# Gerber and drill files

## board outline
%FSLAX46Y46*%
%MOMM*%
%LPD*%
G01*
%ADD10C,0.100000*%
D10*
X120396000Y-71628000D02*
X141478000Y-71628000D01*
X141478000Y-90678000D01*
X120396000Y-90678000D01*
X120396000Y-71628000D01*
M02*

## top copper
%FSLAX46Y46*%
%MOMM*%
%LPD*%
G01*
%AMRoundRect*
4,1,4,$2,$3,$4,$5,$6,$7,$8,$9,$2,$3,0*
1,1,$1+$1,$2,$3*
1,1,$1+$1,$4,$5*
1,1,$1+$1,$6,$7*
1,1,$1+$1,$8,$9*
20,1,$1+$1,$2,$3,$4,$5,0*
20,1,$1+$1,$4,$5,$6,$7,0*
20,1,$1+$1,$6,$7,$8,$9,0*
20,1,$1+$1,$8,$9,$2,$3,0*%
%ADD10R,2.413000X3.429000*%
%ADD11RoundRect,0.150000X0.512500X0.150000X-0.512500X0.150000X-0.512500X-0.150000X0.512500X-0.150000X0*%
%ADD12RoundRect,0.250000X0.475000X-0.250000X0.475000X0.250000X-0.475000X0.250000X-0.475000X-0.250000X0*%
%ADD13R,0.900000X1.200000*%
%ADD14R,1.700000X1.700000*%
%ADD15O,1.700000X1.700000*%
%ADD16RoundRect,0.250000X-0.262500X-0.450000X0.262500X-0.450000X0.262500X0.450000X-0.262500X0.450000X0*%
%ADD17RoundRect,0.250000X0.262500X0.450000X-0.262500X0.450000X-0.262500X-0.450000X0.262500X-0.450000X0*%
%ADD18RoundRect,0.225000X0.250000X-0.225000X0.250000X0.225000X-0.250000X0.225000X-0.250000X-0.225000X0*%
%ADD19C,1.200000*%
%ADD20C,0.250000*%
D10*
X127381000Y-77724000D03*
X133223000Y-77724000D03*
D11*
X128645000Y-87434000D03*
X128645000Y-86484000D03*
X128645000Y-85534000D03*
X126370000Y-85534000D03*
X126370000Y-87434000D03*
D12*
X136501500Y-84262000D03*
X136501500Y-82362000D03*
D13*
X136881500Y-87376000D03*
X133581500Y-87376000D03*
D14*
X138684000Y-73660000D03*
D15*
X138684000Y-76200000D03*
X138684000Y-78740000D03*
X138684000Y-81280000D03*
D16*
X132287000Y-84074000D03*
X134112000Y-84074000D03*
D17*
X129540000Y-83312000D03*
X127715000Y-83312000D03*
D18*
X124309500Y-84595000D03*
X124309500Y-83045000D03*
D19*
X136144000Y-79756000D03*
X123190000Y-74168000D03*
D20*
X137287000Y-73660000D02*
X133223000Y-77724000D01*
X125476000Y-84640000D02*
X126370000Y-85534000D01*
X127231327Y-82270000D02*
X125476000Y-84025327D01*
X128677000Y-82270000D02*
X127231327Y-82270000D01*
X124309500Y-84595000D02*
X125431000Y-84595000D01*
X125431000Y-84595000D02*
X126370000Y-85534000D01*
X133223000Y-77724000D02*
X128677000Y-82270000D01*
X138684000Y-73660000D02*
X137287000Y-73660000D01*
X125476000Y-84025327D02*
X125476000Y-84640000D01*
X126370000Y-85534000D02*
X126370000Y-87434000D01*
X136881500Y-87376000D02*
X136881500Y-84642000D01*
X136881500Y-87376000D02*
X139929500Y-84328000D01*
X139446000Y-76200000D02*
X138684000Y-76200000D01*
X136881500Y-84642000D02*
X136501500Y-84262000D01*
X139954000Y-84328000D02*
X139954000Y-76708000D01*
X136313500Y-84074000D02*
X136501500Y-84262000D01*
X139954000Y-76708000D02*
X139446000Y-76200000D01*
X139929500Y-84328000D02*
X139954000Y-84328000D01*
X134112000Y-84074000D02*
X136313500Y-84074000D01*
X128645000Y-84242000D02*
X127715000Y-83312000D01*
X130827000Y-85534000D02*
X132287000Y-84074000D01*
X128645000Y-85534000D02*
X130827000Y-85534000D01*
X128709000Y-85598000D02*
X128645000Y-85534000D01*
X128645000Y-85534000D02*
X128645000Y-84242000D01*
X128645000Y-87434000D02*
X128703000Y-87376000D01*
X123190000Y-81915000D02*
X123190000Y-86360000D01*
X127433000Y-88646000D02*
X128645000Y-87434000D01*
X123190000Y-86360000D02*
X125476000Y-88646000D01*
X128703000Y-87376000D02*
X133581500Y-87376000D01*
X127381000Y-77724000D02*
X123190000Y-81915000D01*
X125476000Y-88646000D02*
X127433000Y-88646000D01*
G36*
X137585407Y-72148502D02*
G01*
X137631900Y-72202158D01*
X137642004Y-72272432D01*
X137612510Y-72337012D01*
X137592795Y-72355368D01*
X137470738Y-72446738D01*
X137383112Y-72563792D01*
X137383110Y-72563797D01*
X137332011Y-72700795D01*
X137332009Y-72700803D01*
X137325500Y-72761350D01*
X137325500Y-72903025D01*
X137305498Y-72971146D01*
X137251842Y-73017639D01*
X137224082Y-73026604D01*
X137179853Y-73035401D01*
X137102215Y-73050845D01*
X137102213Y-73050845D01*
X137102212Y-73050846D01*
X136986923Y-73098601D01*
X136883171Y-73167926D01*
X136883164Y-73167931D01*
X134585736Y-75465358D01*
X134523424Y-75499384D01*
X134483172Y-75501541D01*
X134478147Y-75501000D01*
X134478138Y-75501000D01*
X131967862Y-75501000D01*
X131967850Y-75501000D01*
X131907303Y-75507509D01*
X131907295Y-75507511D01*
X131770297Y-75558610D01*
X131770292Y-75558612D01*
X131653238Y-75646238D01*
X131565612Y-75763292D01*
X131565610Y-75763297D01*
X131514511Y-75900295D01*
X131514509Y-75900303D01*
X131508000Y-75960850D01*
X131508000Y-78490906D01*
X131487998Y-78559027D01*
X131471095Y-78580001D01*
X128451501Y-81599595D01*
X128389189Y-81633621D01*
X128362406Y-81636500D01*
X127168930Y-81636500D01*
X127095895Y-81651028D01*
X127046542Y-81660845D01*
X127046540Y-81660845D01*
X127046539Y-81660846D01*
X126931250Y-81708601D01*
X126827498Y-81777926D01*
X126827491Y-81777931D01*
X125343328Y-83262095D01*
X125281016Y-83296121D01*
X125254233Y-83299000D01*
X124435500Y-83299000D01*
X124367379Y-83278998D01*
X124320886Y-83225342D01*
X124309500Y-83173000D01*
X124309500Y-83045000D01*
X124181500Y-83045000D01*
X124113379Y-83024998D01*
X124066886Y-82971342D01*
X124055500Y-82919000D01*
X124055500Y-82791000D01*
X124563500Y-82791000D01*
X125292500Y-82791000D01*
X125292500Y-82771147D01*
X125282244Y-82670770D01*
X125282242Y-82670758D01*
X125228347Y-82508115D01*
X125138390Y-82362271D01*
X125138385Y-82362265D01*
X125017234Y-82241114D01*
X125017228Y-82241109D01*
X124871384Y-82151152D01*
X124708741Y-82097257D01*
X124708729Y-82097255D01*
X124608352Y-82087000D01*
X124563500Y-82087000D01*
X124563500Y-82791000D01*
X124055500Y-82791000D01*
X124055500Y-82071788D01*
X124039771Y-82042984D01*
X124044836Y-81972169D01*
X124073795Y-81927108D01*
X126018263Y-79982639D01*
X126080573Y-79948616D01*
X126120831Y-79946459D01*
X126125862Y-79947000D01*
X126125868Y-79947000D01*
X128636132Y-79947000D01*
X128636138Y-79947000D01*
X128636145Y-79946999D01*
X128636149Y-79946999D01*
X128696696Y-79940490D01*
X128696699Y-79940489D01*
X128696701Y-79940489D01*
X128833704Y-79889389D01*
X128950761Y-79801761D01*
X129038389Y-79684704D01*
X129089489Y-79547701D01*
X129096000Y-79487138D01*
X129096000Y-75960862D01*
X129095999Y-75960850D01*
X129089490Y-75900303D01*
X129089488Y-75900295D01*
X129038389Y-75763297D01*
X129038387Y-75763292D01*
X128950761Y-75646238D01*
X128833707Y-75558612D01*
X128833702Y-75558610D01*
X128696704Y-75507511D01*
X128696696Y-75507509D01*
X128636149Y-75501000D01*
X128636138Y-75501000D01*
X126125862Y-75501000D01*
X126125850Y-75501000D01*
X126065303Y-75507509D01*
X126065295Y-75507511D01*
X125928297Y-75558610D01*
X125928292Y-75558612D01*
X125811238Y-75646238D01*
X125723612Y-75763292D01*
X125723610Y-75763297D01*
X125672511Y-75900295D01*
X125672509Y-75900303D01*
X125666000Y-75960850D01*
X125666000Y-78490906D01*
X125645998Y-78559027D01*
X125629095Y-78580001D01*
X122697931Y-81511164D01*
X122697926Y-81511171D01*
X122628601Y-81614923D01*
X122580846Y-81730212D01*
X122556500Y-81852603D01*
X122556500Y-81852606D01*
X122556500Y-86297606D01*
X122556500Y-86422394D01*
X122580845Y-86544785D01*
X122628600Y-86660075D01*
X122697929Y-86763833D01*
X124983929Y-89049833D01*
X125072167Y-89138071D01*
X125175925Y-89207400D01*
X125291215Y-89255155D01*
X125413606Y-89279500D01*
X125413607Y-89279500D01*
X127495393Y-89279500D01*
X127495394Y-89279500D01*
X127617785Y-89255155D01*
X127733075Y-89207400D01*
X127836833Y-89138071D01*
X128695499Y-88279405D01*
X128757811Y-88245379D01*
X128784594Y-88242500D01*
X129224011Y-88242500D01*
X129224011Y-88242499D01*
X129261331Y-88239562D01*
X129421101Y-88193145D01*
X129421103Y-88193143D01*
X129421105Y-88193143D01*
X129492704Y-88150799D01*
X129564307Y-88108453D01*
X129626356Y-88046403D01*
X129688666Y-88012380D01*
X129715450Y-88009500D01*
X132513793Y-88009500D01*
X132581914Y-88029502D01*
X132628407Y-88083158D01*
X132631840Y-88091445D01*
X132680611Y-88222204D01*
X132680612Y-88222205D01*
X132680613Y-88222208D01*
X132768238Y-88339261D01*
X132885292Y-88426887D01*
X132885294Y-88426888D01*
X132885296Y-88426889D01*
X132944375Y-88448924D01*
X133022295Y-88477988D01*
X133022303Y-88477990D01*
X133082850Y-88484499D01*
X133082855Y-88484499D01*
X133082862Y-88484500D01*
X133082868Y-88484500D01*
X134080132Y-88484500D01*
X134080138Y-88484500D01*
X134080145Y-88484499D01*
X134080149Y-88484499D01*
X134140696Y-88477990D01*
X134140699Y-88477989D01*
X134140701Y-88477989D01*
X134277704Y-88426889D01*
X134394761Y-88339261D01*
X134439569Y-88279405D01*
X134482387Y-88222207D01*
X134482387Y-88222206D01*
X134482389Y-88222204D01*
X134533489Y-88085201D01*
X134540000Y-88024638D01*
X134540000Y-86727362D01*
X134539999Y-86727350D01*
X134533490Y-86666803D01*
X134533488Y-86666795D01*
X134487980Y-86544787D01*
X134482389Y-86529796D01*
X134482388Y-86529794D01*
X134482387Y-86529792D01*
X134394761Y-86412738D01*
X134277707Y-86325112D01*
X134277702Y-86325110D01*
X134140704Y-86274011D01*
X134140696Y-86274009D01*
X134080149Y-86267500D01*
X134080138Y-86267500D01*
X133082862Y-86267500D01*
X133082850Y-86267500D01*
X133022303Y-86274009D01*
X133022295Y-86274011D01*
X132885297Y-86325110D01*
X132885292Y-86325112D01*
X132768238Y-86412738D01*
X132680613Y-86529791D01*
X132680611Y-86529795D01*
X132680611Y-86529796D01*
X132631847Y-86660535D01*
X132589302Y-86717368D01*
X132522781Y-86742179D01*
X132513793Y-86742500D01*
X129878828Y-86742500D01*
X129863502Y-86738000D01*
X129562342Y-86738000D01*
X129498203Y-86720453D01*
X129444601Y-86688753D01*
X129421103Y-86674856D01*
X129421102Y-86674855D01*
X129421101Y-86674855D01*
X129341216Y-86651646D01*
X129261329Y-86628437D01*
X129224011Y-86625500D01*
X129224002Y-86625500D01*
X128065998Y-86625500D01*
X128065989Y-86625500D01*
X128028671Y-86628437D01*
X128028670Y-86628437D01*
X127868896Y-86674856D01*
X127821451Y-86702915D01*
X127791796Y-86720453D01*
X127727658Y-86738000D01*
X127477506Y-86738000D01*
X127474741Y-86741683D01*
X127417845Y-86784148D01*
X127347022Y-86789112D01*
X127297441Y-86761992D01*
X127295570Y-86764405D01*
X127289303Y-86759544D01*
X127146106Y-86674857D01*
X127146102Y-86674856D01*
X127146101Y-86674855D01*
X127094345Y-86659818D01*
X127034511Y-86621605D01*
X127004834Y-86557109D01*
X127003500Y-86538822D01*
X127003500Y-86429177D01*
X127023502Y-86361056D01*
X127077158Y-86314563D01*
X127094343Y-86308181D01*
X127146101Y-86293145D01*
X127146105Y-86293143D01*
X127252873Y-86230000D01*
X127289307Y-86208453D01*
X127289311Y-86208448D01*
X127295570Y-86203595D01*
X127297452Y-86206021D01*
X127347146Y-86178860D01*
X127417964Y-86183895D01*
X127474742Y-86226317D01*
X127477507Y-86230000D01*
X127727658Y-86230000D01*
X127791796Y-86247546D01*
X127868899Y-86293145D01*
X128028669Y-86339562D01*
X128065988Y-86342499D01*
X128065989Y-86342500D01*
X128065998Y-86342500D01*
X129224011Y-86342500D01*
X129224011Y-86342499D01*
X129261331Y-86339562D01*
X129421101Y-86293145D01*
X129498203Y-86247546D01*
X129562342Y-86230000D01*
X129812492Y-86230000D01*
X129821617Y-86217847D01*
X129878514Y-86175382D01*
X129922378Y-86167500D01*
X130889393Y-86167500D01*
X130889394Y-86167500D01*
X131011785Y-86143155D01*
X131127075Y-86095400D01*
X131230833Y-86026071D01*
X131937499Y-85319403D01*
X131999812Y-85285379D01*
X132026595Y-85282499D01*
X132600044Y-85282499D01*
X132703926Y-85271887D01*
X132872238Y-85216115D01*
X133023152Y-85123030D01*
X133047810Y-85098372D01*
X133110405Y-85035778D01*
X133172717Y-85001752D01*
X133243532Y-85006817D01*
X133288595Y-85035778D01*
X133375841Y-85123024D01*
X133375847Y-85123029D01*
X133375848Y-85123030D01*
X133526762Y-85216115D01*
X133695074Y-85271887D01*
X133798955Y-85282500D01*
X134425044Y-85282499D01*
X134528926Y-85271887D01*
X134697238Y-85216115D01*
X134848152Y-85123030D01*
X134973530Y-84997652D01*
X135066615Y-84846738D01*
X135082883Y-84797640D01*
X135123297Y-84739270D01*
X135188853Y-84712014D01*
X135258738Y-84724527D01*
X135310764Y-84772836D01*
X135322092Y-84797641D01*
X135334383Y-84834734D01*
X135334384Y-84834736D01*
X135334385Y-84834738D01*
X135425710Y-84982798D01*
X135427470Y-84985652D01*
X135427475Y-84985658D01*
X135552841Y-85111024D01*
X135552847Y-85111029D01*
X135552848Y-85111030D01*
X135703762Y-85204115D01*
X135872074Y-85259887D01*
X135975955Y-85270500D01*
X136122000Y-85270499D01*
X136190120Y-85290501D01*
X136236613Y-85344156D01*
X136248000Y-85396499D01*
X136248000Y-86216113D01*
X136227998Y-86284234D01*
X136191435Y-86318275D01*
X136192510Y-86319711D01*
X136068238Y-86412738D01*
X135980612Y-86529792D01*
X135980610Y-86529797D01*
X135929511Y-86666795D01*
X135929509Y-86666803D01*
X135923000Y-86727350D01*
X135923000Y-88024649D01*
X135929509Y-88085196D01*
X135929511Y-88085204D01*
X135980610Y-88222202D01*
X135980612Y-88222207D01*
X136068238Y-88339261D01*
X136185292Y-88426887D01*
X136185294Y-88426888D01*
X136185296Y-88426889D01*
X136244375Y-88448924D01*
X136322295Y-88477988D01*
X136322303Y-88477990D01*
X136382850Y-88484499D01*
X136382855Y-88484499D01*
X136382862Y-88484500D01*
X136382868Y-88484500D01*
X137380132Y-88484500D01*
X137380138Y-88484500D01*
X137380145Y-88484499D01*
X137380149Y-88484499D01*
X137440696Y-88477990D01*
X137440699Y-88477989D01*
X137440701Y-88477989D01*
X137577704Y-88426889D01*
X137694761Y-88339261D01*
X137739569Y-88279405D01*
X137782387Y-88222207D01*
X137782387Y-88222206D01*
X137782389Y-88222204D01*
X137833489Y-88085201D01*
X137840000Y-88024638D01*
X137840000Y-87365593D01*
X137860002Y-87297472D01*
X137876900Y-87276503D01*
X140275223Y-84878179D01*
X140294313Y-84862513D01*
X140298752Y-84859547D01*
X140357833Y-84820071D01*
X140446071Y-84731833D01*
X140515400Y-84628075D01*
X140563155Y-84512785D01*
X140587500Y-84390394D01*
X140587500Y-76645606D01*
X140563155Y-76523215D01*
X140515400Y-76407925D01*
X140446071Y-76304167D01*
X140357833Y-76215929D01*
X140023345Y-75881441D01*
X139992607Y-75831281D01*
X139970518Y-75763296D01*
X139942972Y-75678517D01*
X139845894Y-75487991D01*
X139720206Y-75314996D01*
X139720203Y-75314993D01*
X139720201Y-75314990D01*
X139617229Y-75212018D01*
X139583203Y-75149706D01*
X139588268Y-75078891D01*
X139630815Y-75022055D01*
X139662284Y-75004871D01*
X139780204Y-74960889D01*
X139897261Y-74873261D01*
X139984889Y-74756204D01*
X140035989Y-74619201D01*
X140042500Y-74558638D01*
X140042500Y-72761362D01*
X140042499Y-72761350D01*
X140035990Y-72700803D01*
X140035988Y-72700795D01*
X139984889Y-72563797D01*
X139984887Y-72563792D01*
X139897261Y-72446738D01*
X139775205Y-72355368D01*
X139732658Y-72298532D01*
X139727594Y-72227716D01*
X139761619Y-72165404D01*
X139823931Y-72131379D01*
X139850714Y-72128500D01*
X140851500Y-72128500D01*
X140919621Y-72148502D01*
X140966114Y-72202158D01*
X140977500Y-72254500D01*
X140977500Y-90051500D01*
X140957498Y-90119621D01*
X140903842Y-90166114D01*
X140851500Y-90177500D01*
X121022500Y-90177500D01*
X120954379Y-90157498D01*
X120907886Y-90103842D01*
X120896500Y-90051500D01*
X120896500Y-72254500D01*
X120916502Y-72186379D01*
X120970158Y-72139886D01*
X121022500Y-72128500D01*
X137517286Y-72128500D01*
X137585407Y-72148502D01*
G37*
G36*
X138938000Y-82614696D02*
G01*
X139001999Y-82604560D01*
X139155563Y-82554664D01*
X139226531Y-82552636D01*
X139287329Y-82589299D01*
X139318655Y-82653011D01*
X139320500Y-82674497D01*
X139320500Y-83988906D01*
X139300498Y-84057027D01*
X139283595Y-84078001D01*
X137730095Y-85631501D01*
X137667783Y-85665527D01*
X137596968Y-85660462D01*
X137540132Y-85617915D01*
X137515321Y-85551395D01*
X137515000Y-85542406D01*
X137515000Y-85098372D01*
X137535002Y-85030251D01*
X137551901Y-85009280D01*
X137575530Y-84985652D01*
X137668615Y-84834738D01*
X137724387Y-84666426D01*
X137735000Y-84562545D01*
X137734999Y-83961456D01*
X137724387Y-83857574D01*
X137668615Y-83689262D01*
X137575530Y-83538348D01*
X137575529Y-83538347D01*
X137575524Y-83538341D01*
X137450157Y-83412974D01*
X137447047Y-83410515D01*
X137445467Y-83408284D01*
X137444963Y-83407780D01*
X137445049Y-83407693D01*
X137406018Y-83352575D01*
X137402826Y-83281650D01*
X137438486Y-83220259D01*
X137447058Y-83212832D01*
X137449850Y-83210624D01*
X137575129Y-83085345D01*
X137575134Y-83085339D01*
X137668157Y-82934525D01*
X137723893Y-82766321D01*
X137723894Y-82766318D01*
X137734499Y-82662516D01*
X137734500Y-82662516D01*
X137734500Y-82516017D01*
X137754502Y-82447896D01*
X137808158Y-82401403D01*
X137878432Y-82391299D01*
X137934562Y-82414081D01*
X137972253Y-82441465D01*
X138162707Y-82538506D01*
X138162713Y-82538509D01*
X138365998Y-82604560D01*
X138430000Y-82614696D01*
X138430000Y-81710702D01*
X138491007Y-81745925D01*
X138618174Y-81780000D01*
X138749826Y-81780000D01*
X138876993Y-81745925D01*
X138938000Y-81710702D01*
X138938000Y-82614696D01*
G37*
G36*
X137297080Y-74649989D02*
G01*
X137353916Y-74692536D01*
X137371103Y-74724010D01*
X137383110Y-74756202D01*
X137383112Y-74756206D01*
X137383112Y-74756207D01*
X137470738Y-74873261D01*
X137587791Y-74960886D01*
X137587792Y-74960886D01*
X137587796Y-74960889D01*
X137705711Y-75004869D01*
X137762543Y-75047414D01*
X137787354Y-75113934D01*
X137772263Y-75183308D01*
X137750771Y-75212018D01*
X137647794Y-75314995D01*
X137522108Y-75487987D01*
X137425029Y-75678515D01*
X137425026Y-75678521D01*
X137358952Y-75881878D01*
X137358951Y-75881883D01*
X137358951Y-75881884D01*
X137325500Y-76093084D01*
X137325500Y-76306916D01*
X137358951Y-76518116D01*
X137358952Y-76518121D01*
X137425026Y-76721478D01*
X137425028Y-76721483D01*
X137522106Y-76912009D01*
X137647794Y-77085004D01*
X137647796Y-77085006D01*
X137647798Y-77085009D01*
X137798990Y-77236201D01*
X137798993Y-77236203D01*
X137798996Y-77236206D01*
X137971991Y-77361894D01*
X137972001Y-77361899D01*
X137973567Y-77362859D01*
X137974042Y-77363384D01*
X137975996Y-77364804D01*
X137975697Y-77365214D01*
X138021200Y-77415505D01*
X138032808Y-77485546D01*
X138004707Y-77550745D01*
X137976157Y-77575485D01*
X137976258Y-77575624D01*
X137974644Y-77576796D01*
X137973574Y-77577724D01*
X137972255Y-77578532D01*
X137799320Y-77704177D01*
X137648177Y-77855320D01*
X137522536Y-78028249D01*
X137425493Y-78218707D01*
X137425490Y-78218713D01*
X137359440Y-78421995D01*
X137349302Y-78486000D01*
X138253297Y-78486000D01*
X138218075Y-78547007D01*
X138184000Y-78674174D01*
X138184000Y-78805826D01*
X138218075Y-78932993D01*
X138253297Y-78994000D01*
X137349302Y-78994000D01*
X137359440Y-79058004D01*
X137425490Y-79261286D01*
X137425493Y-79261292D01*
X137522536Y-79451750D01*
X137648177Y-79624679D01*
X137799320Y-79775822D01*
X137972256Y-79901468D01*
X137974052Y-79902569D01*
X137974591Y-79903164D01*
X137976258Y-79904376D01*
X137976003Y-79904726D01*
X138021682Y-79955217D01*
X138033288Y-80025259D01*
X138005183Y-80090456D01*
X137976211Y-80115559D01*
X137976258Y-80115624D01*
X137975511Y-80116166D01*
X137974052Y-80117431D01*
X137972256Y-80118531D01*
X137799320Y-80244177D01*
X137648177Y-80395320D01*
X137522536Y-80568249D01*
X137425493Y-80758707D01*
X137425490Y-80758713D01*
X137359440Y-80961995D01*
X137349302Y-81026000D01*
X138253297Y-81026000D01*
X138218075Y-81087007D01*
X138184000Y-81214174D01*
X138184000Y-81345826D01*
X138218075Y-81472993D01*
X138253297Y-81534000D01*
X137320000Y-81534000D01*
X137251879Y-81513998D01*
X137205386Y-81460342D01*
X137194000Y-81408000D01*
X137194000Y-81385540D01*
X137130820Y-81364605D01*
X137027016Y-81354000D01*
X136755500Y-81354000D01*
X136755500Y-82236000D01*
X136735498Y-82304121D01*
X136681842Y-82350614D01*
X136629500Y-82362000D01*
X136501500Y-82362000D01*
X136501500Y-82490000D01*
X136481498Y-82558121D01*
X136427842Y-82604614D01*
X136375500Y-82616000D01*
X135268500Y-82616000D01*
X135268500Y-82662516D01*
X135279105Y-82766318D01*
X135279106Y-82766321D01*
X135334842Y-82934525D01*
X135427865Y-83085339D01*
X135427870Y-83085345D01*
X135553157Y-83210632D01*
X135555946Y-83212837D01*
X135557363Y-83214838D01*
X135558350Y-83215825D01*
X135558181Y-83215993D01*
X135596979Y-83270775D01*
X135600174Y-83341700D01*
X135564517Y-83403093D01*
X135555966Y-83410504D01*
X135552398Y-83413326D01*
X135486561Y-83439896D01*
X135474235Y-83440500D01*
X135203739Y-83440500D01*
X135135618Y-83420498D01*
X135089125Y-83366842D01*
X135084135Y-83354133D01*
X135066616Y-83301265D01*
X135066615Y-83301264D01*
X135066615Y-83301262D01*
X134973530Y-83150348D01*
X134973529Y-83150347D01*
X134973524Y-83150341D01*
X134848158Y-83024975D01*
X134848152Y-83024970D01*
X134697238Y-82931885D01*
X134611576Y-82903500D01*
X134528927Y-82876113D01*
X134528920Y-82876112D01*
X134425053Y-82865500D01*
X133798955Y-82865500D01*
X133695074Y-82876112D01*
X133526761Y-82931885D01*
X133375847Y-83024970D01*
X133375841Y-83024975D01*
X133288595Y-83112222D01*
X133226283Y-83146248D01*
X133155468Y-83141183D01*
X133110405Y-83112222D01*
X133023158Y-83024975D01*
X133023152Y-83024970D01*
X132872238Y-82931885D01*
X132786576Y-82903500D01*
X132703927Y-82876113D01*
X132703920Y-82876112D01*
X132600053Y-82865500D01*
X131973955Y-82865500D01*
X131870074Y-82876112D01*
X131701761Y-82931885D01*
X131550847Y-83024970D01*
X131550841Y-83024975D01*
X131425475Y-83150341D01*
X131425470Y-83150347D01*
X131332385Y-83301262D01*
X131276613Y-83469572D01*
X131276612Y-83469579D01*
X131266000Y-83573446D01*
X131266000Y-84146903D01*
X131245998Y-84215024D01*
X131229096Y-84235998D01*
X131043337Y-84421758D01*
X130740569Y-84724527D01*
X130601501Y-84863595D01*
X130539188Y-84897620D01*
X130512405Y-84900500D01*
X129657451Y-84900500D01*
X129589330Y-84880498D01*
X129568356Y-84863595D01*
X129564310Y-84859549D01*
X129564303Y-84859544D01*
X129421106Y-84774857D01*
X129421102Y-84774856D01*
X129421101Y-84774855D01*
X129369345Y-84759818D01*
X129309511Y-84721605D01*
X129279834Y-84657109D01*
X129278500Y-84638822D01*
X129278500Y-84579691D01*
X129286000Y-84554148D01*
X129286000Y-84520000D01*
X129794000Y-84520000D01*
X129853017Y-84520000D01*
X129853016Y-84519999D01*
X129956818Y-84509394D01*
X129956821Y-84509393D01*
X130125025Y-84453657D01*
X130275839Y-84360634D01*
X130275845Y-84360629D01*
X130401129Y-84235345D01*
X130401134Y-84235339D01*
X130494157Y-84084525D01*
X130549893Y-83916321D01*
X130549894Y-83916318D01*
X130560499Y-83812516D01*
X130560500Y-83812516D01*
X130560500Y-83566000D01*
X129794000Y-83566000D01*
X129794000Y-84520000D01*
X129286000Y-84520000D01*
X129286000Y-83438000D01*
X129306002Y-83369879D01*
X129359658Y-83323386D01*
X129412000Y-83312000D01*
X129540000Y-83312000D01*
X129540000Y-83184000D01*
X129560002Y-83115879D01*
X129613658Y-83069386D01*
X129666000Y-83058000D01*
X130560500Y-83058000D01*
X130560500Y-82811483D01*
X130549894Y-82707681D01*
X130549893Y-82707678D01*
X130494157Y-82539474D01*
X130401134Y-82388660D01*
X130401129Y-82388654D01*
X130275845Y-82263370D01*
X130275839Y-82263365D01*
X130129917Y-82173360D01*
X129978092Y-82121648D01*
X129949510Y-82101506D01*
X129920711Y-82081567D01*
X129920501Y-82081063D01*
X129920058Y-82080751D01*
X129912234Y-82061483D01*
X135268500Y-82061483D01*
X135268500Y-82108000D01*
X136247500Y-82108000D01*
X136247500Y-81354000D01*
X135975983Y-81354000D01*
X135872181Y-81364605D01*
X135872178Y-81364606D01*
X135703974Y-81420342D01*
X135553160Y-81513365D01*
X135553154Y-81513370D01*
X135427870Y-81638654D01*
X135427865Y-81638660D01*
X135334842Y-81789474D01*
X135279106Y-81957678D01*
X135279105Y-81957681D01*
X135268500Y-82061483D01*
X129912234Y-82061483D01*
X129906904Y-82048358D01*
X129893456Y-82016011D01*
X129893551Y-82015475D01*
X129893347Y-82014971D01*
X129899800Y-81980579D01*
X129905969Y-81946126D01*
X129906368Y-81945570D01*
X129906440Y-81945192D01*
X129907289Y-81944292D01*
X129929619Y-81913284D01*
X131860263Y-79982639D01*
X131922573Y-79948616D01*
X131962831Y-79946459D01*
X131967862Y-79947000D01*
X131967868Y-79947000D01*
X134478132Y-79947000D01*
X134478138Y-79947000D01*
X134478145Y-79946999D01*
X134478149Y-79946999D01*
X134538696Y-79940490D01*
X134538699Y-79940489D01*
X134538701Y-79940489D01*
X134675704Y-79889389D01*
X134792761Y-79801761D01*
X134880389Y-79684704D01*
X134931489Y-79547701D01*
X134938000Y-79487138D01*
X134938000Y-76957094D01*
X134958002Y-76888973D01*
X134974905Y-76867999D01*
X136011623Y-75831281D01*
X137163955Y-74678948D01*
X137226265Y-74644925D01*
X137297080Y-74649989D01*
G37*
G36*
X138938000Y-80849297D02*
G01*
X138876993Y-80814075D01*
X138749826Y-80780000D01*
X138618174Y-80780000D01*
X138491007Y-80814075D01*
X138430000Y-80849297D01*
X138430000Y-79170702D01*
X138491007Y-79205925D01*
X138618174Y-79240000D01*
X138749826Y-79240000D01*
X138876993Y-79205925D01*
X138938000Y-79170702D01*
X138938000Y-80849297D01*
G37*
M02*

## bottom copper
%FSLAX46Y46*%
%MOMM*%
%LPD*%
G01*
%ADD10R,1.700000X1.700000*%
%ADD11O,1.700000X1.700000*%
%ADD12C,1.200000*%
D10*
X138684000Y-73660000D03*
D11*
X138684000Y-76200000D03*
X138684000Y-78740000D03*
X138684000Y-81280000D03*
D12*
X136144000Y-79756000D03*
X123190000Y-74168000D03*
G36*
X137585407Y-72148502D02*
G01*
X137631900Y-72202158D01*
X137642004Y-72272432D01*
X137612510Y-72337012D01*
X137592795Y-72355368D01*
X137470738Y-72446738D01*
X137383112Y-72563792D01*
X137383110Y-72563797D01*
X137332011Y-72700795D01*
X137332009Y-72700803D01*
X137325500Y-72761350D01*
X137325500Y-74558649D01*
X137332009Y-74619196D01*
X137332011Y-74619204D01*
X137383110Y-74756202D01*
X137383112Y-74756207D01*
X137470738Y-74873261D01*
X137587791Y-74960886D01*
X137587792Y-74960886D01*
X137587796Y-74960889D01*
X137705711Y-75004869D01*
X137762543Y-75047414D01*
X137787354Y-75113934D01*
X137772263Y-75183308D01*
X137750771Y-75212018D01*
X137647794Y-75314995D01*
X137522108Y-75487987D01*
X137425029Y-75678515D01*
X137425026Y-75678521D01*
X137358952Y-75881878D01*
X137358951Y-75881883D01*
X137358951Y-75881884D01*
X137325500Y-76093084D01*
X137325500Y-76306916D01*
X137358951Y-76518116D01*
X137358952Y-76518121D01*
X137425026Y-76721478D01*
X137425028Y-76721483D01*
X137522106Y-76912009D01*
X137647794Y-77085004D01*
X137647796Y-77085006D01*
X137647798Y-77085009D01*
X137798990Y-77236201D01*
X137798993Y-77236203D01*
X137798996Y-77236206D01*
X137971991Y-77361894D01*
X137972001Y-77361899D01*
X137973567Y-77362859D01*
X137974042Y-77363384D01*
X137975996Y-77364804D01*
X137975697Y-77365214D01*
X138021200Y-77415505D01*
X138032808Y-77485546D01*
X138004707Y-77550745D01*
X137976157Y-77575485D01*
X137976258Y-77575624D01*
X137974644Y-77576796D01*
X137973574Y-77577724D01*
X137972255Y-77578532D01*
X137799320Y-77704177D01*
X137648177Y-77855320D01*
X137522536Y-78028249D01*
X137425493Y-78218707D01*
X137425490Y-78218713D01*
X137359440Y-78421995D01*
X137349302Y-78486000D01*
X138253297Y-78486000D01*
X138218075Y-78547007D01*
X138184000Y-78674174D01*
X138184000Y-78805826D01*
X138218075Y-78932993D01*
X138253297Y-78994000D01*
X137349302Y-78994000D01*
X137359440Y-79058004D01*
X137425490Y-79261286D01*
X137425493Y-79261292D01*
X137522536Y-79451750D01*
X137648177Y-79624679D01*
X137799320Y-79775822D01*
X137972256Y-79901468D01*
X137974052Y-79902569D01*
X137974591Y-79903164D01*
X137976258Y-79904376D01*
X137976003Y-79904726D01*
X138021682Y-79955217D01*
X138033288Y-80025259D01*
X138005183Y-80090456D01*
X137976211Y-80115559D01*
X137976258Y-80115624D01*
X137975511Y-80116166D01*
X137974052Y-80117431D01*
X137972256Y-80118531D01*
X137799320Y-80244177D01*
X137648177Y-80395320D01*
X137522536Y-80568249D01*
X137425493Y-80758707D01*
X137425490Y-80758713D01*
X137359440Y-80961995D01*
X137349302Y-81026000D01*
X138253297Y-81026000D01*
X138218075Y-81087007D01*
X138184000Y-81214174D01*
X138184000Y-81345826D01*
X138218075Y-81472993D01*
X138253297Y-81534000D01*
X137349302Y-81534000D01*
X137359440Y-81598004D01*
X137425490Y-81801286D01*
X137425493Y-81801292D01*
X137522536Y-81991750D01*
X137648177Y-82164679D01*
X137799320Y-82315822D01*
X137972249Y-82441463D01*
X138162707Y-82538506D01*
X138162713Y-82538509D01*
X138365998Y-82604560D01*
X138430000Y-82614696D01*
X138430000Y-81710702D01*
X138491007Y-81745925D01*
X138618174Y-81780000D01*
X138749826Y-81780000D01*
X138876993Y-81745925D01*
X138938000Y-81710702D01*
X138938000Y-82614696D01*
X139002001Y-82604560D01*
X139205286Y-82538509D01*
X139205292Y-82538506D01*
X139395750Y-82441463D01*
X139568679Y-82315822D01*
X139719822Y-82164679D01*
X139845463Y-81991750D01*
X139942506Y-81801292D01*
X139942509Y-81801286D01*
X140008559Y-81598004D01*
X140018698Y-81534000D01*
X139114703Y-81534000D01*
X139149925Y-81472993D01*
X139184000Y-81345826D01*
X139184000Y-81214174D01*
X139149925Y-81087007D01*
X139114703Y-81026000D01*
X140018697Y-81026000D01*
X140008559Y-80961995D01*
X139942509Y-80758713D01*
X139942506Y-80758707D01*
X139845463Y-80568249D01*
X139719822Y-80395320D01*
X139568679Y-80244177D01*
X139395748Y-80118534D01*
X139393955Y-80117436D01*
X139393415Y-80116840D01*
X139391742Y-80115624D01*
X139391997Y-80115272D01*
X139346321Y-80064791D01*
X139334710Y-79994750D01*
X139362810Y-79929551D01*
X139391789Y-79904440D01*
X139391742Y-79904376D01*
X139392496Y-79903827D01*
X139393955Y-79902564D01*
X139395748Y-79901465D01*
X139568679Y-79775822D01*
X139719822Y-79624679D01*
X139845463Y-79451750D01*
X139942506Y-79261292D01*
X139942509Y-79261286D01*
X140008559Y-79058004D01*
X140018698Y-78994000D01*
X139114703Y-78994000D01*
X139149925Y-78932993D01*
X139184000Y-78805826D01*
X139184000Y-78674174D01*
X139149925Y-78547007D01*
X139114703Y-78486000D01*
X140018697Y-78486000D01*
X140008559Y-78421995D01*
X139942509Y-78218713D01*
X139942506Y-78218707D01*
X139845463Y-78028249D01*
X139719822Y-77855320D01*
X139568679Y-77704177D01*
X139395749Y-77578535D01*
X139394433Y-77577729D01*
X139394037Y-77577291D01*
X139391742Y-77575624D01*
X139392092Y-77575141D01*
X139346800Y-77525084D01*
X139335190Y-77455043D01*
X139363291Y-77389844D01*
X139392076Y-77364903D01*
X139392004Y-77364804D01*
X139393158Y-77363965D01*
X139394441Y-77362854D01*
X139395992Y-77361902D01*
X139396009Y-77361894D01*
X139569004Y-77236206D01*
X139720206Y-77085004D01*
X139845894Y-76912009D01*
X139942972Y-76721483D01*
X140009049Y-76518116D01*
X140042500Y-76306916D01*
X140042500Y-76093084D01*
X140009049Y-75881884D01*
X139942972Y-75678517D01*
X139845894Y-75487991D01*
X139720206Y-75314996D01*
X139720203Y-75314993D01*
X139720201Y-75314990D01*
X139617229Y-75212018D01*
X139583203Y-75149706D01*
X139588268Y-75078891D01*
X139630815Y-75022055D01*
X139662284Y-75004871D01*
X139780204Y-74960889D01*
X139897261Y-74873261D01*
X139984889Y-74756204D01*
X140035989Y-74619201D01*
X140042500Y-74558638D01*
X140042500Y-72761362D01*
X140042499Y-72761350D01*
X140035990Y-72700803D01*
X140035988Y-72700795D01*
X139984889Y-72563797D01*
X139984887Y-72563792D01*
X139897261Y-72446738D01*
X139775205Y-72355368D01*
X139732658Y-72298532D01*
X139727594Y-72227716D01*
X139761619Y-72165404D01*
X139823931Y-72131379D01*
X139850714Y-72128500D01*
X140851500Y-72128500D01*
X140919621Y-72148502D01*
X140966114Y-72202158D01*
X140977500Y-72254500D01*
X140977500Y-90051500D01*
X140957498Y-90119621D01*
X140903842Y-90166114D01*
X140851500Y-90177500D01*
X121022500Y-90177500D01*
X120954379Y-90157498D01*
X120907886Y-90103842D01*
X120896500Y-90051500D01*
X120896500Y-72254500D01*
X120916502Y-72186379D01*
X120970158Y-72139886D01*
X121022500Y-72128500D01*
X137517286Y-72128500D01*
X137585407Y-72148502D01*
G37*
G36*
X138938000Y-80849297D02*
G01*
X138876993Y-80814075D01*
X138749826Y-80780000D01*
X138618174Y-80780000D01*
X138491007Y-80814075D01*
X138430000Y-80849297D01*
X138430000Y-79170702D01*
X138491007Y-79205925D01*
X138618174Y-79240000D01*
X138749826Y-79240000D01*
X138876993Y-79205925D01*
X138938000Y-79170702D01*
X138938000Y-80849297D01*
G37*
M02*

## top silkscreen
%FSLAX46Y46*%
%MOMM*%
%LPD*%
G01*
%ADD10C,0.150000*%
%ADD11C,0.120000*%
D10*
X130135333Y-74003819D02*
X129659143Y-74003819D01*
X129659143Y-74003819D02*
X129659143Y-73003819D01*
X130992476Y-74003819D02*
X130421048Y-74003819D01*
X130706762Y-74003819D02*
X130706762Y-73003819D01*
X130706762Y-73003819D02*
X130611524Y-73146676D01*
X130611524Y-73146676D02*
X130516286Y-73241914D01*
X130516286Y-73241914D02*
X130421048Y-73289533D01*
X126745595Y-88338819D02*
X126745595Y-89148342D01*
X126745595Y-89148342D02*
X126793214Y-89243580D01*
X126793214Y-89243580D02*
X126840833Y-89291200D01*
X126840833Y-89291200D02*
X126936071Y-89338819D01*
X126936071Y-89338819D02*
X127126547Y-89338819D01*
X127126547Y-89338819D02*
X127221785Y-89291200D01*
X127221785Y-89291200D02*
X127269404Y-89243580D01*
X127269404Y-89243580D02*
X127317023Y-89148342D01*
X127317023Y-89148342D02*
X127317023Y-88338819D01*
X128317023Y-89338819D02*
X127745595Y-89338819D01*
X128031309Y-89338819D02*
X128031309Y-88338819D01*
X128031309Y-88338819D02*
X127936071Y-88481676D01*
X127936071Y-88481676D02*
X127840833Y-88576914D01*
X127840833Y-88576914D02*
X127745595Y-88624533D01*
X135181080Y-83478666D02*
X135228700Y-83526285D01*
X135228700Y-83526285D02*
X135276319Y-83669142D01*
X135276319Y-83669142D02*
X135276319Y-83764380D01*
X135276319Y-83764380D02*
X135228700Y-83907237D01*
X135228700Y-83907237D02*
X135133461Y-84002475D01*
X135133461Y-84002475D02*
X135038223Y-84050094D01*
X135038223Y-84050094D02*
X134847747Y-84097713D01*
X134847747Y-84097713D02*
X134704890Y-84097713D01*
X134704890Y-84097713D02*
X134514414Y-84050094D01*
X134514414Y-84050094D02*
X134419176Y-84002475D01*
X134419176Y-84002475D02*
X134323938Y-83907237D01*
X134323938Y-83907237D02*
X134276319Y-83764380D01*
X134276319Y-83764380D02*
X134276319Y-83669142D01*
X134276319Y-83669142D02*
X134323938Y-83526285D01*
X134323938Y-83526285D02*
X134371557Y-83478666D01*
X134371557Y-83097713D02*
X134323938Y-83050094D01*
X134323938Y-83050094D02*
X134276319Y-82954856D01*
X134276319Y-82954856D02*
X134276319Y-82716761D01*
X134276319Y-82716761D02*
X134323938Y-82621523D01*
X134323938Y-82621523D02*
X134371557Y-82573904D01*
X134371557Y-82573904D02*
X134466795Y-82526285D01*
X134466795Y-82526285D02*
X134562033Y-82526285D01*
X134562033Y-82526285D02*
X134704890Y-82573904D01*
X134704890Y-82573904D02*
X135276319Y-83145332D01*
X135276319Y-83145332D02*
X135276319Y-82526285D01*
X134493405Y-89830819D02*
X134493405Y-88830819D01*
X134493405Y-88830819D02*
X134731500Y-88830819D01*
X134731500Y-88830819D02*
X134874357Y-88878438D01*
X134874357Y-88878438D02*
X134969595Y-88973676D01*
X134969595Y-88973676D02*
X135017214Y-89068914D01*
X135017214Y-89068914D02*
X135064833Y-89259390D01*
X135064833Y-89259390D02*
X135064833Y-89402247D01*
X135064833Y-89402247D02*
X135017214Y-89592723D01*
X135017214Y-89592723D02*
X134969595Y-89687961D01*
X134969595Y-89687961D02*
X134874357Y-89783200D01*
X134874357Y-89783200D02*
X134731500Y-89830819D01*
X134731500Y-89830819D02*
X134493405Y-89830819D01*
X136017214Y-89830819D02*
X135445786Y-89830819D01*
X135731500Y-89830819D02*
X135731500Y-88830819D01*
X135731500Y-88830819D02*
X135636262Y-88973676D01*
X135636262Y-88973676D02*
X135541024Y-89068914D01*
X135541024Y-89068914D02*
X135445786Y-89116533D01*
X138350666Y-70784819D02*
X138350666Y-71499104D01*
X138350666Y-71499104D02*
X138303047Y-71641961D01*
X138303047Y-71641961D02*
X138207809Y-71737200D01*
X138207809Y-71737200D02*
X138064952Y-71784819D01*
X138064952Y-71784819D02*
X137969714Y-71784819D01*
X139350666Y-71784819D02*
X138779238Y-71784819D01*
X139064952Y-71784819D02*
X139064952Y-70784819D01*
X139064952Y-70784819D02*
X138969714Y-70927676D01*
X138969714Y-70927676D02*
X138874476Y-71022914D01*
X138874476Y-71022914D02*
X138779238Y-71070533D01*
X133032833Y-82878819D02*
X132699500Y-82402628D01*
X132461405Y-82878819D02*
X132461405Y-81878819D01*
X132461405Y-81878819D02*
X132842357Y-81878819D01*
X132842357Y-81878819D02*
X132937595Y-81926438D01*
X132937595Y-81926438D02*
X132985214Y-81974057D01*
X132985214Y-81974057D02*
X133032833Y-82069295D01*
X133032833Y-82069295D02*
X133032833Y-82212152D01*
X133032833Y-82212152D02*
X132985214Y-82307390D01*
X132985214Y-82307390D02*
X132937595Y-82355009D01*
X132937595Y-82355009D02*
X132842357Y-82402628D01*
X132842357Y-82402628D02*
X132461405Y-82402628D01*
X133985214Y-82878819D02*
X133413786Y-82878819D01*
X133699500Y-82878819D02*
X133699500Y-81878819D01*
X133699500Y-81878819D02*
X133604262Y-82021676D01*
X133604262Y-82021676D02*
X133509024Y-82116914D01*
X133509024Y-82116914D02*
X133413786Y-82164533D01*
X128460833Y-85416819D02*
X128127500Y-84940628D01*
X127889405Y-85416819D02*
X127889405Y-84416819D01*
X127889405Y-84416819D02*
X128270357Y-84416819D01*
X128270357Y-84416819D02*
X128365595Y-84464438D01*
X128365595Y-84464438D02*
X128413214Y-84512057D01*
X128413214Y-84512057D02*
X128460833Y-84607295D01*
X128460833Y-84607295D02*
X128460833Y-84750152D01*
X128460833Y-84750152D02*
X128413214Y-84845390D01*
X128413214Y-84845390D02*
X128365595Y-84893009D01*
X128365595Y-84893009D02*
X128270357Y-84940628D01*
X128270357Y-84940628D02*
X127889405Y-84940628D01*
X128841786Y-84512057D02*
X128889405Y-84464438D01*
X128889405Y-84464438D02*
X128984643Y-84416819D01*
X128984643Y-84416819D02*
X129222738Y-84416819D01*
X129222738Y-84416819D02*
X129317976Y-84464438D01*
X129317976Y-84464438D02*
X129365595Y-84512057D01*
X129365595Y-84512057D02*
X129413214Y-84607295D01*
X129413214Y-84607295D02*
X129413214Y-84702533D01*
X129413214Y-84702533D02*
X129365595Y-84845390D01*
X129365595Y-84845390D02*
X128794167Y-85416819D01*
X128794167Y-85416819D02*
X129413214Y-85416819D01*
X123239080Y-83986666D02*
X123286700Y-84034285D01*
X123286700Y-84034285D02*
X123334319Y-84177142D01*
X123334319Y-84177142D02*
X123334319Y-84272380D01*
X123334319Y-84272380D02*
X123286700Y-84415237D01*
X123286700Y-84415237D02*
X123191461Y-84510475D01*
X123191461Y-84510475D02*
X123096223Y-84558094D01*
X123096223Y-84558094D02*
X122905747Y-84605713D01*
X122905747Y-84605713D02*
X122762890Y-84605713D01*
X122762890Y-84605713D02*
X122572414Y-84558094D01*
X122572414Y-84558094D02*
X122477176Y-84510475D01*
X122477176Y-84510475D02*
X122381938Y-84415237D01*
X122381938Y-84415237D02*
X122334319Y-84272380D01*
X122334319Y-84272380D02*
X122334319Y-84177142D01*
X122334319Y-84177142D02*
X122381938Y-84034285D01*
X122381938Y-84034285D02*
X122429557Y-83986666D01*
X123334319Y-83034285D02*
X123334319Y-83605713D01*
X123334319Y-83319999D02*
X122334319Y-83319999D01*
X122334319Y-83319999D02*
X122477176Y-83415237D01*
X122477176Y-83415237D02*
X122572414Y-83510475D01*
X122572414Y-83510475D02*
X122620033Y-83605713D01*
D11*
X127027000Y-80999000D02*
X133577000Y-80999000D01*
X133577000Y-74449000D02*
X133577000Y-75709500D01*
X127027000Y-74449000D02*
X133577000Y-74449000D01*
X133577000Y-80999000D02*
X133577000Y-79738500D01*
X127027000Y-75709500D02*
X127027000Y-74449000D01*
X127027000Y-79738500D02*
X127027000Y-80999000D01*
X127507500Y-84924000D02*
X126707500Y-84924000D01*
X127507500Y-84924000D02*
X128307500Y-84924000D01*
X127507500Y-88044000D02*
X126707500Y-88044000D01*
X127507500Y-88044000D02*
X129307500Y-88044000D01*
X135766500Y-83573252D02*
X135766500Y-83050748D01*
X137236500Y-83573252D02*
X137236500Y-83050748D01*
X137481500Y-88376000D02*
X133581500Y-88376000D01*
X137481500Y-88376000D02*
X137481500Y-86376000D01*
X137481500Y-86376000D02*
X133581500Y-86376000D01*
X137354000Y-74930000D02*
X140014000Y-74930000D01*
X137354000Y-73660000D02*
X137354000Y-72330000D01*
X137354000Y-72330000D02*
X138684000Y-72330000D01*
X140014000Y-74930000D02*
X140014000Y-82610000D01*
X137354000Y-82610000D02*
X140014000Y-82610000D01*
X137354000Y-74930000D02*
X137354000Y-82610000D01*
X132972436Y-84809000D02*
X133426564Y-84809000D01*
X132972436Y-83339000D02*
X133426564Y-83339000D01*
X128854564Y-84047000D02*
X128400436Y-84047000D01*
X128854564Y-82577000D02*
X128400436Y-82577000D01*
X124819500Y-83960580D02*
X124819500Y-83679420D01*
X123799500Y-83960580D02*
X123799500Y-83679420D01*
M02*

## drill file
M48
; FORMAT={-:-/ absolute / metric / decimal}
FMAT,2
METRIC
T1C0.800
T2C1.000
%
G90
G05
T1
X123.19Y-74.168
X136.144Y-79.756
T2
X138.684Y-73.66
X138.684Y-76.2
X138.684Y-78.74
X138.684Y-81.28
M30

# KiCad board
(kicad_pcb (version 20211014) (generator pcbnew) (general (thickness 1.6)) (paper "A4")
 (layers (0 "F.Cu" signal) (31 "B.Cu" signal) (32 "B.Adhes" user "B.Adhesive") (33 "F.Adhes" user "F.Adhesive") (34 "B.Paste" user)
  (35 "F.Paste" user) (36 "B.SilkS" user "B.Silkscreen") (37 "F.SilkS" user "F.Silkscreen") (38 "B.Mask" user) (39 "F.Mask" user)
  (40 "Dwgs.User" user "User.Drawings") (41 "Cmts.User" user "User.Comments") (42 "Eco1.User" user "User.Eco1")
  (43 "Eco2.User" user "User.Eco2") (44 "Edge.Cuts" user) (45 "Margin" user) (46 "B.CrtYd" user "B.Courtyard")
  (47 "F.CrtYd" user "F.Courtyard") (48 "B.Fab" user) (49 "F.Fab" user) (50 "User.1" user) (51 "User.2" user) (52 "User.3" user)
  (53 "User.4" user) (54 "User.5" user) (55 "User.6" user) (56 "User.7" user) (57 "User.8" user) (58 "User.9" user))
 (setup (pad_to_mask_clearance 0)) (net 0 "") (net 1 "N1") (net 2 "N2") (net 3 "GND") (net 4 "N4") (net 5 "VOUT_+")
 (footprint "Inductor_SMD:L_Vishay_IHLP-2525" (layer "F.Cu") (at 130.302 77.724)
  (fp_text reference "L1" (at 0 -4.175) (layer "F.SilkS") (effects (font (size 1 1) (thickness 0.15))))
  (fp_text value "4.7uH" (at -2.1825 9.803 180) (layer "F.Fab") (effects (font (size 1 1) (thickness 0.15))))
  (fp_line (start -3.275 3.275) (end 3.275 3.275) (layer "F.SilkS") (width 0.12))
  (fp_line (start 3.275 -3.275) (end 3.275 -2.0145) (layer "F.SilkS") (width 0.12))
  (fp_line (start -3.275 -3.275) (end 3.275 -3.275) (layer "F.SilkS") (width 0.12))
  (fp_line (start 3.275 3.275) (end 3.275 2.0145) (layer "F.SilkS") (width 0.12))
  (fp_line (start -3.275 -2.0145) (end -3.275 -3.275) (layer "F.SilkS") (width 0.12))
  (fp_line (start -3.275 2.0145) (end -3.275 3.275) (layer "F.SilkS") (width 0.12))
  (pad "1" smd rect (at -2.921 0) (size 2.413 3.429) (layers "F.Cu" "F.Paste" "F.Mask") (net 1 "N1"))
  (pad "2" smd rect (at 2.921 0) (size 2.413 3.429) (layers "F.Cu" "F.Paste" "F.Mask") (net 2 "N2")))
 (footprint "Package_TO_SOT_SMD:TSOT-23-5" (layer "F.Cu") (at 127.5075 86.484 180)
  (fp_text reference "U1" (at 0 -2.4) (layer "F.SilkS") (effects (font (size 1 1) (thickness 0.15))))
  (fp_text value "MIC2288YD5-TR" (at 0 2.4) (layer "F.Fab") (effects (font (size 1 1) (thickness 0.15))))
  (fp_line (start 0 1.56) (end 0.8 1.56) (layer "F.SilkS") (width 0.12))
  (fp_line (start 0 1.56) (end -0.8 1.56) (layer "F.SilkS") (width 0.12))
  (fp_line (start 0 -1.56) (end 0.8 -1.56) (layer "F.SilkS") (width 0.12))
  (fp_line (start 0 -1.56) (end -1.8 -1.56) (layer "F.SilkS") (width 0.12))
  (pad "1" smd roundrect (at -1.1375 -0.95 180) (size 1.325 0.6) (layers "F.Cu" "F.Paste" "F.Mask") (roundrect_rratio 0.25) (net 1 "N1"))
  (pad "2" smd roundrect (at -1.1375 0 180) (size 1.325 0.6) (layers "F.Cu" "F.Paste" "F.Mask") (roundrect_rratio 0.25) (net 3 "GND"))
  (pad "3" smd roundrect (at -1.1375 0.95 180) (size 1.325 0.6) (layers "F.Cu" "F.Paste" "F.Mask") (roundrect_rratio 0.25) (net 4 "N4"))
  (pad "4" smd roundrect (at 1.1375 0.95 180) (size 1.325 0.6) (layers "F.Cu" "F.Paste" "F.Mask") (roundrect_rratio 0.25) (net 2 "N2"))
  (pad "5" smd roundrect (at 1.1375 -0.95 180) (size 1.325 0.6) (layers "F.Cu" "F.Paste" "F.Mask") (roundrect_rratio 0.25) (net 2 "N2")))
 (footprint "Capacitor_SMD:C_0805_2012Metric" (layer "F.Cu") (at 136.5015 83.312 90)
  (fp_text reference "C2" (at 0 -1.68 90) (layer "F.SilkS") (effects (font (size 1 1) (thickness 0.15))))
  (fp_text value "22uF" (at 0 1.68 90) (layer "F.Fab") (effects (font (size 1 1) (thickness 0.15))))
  (fp_line (start -0.261252 -0.735) (end 0.261252 -0.735) (layer "F.SilkS") (width 0.12))
  (fp_line (start -0.261252 0.735) (end 0.261252 0.735) (layer "F.SilkS") (width 0.12))
  (pad "1" smd roundrect (at -0.95 0 90) (size 1 1.45) (layers "F.Cu" "F.Paste" "F.Mask") (roundrect_rratio 0.25) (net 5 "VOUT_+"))
  (pad "2" smd roundrect (at 0.95 0 90) (size 1 1.45) (layers "F.Cu" "F.Paste" "F.Mask") (roundrect_rratio 0.25) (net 3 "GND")))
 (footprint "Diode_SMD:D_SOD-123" (layer "F.Cu") (at 135.2315 87.376 180)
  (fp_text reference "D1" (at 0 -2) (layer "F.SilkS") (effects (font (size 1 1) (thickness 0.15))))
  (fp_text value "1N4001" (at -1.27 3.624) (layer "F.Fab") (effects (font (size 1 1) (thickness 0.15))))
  (fp_line (start -2.25 -1) (end 1.65 -1) (layer "F.SilkS") (width 0.12))
  (fp_line (start -2.25 -1) (end -2.25 1) (layer "F.SilkS") (width 0.12))
  (fp_line (start -2.25 1) (end 1.65 1) (layer "F.SilkS") (width 0.12))
  (pad "1" smd rect (at -1.65 0 180) (size 0.9 1.2) (layers "F.Cu" "F.Paste" "F.Mask") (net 5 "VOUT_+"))
  (pad "2" smd rect (at 1.65 0 180) (size 0.9 1.2) (layers "F.Cu" "F.Paste" "F.Mask") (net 1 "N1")))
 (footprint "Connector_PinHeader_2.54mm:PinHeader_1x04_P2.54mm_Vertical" (layer "F.Cu") (at 138.684 73.66)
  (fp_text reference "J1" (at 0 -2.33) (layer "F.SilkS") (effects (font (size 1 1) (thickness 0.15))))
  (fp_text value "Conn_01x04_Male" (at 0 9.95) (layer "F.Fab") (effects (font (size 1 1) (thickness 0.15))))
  (fp_line (start -1.33 1.27) (end 1.33 1.27) (layer "F.SilkS") (width 0.12))
  (fp_line (start -1.33 0) (end -1.33 -1.33) (layer "F.SilkS") (width 0.12))
  (fp_line (start -1.33 -1.33) (end 0 -1.33) (layer "F.SilkS") (width 0.12))
  (fp_line (start 1.33 1.27) (end 1.33 8.95) (layer "F.SilkS") (width 0.12))
  (fp_line (start -1.33 8.95) (end 1.33 8.95) (layer "F.SilkS") (width 0.12))
  (fp_line (start -1.33 1.27) (end -1.33 8.95) (layer "F.SilkS") (width 0.12))
  (pad "1" thru_hole rect (at 0 0) (size 1.7 1.7) (drill 1) (layers *.Cu *.Mask) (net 2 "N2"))
  (pad "2" thru_hole oval (at 0 2.54) (size 1.7 1.7) (drill 1) (layers *.Cu *.Mask) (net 5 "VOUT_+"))
  (pad "3" thru_hole oval (at 0 5.08) (size 1.7 1.7) (drill 1) (layers *.Cu *.Mask) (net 3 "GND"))
  (pad "4" thru_hole oval (at 0 7.62) (size 1.7 1.7) (drill 1) (layers *.Cu *.Mask) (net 3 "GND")))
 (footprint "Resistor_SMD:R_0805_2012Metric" (layer "F.Cu") (at 133.1995 84.074)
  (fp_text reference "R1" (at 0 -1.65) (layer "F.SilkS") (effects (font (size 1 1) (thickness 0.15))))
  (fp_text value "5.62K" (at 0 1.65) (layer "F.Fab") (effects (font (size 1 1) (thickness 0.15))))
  (fp_line (start -0.227064 0.735) (end 0.227064 0.735) (layer "F.SilkS") (width 0.12))
  (fp_line (start -0.227064 -0.735) (end 0.227064 -0.735) (layer "F.SilkS") (width 0.12))
  (pad "1" smd roundrect (at -0.9125 0) (size 1.025 1.4) (layers "F.Cu" "F.Paste" "F.Mask") (roundrect_rratio 0.243902439) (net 4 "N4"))
  (pad "2" smd roundrect (at 0.9125 0) (size 1.025 1.4) (layers "F.Cu" "F.Paste" "F.Mask") (roundrect_rratio 0.243902439) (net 5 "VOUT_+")))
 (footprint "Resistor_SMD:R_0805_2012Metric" (layer "F.Cu") (at 128.6275 83.312 180)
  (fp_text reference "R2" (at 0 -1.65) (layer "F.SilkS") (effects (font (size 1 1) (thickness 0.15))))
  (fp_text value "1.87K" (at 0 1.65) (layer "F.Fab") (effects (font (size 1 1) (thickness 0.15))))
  (fp_line (start -0.227064 -0.735) (end 0.227064 -0.735) (layer "F.SilkS") (width 0.12))
  (fp_line (start -0.227064 0.735) (end 0.227064 0.735) (layer "F.SilkS") (width 0.12))
  (pad "1" smd roundrect (at -0.9125 0 180) (size 1.025 1.4) (layers "F.Cu" "F.Paste" "F.Mask") (roundrect_rratio 0.243902439) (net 3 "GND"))
  (pad "2" smd roundrect (at 0.9125 0 180) (size 1.025 1.4) (layers "F.Cu" "F.Paste" "F.Mask") (roundrect_rratio 0.243902439) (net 4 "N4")))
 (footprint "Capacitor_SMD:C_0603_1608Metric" (layer "F.Cu") (at 124.3095 83.82 90)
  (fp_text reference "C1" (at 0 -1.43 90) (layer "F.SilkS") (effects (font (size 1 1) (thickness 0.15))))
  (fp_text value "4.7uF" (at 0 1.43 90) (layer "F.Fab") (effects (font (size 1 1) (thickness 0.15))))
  (fp_line (start -0.14058 0.51) (end 0.14058 0.51) (layer "F.SilkS") (width 0.12))
  (fp_line (start -0.14058 -0.51) (end 0.14058 -0.51) (layer "F.SilkS") (width 0.12))
  (pad "1" smd roundrect (at -0.775 0 90) (size 0.9 0.95) (layers "F.Cu" "F.Paste" "F.Mask") (roundrect_rratio 0.25) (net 2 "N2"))
  (pad "2" smd roundrect (at 0.775 0 90) (size 0.9 0.95) (layers "F.Cu" "F.Paste" "F.Mask") (roundrect_rratio 0.25) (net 3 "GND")))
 (gr_rect (start 120.396 71.628) (end 141.478 90.678) (layer "Edge.Cuts") (width 0.1) (fill none))
 (segment (start 137.287 73.66) (end 133.223 77.724) (width 0.25) (layer "F.Cu") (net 2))
 (segment (start 125.476 84.64) (end 126.37 85.534) (width 0.25) (layer "F.Cu") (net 2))
 (segment (start 127.231327 82.27) (end 125.476 84.025327) (width 0.25) (layer "F.Cu") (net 2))
 (segment (start 128.677 82.27) (end 127.231327 82.27) (width 0.25) (layer "F.Cu") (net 2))
 (segment (start 124.3095 84.595) (end 125.431 84.595) (width 0.25) (layer "F.Cu") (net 2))
 (segment (start 125.431 84.595) (end 126.37 85.534) (width 0.25) (layer "F.Cu") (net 2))
 (segment (start 133.223 77.724) (end 128.677 82.27) (width 0.25) (layer "F.Cu") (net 2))
 (segment (start 138.684 73.66) (end 137.287 73.66) (width 0.25) (layer "F.Cu") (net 2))
 (segment (start 125.476 84.025327) (end 125.476 84.64) (width 0.25) (layer "F.Cu") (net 2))
 (segment (start 126.37 85.534) (end 126.37 87.434) (width 0.25) (layer "F.Cu") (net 2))
 (via (at 136.144 79.756) (size 1.2) (drill 0.8) (layers "F.Cu" "B.Cu") (free) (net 3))
 (via (at 123.19 74.168) (size 1.2) (drill 0.8) (layers "F.Cu" "B.Cu") (free) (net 3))
 (segment (start 136.8815 87.376) (end 136.8815 84.642) (width 0.25) (layer "F.Cu") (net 5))
 (segment (start 136.8815 87.376) (end 139.9295 84.328) (width 0.25) (layer "F.Cu") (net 5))
 (segment (start 139.446 76.2) (end 138.684 76.2) (width 0.25) (layer "F.Cu") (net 5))
 (segment (start 136.8815 84.642) (end 136.5015 84.262) (width 0.25) (layer "F.Cu") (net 5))
 (segment (start 139.954 84.328) (end 139.954 76.708) (width 0.25) (layer "F.Cu") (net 5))
 (segment (start 136.3135 84.074) (end 136.5015 84.262) (width 0.25) (layer "F.Cu") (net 5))
 (segment (start 139.954 76.708) (end 139.446 76.2) (width 0.25) (layer "F.Cu") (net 5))
 (segment (start 139.9295 84.328) (end 139.954 84.328) (width 0.25) (layer "F.Cu") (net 5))
 (segment (start 134.112 84.074) (end 136.3135 84.074) (width 0.25) (layer "F.Cu") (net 5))
 (segment (start 128.645 84.242) (end 127.715 83.312) (width 0.25) (layer "F.Cu") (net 4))
 (segment (start 130.827 85.534) (end 132.287 84.074) (width 0.25) (layer "F.Cu") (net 4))
 (segment (start 128.645 85.534) (end 130.827 85.534) (width 0.25) (layer "F.Cu") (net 4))
 (segment (start 128.709 85.598) (end 128.645 85.534) (width 0.25) (layer "F.Cu") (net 4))
 (segment (start 128.645 85.534) (end 128.645 84.242) (width 0.25) (layer "F.Cu") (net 4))
 (segment (start 128.645 87.434) (end 128.703 87.376) (width 0.25) (layer "F.Cu") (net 1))
 (segment (start 123.19 81.915) (end 123.19 86.36) (width 0.25) (layer "F.Cu") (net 1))
 (segment (start 127.433 88.646) (end 128.645 87.434) (width 0.25) (layer "F.Cu") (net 1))
 (segment (start 123.19 86.36) (end 125.476 88.646) (width 0.25) (layer "F.Cu") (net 1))
 (segment (start 128.703 87.376) (end 133.5815 87.376) (width 0.25) (layer "F.Cu") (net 1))
 (segment (start 127.381 77.724) (end 123.19 81.915) (width 0.25) (layer "F.Cu") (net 1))
 (segment (start 125.476 88.646) (end 127.433 88.646) (width 0.25) (layer "F.Cu") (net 1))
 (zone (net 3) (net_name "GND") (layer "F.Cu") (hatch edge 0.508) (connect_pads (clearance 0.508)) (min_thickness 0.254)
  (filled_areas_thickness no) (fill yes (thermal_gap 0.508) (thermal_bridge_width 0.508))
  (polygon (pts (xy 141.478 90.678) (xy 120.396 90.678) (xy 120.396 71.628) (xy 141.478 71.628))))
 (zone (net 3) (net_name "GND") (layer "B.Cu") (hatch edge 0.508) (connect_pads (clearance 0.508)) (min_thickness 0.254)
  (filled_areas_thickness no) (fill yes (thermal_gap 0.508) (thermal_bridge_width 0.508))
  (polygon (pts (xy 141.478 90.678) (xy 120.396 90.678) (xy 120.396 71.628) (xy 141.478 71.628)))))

